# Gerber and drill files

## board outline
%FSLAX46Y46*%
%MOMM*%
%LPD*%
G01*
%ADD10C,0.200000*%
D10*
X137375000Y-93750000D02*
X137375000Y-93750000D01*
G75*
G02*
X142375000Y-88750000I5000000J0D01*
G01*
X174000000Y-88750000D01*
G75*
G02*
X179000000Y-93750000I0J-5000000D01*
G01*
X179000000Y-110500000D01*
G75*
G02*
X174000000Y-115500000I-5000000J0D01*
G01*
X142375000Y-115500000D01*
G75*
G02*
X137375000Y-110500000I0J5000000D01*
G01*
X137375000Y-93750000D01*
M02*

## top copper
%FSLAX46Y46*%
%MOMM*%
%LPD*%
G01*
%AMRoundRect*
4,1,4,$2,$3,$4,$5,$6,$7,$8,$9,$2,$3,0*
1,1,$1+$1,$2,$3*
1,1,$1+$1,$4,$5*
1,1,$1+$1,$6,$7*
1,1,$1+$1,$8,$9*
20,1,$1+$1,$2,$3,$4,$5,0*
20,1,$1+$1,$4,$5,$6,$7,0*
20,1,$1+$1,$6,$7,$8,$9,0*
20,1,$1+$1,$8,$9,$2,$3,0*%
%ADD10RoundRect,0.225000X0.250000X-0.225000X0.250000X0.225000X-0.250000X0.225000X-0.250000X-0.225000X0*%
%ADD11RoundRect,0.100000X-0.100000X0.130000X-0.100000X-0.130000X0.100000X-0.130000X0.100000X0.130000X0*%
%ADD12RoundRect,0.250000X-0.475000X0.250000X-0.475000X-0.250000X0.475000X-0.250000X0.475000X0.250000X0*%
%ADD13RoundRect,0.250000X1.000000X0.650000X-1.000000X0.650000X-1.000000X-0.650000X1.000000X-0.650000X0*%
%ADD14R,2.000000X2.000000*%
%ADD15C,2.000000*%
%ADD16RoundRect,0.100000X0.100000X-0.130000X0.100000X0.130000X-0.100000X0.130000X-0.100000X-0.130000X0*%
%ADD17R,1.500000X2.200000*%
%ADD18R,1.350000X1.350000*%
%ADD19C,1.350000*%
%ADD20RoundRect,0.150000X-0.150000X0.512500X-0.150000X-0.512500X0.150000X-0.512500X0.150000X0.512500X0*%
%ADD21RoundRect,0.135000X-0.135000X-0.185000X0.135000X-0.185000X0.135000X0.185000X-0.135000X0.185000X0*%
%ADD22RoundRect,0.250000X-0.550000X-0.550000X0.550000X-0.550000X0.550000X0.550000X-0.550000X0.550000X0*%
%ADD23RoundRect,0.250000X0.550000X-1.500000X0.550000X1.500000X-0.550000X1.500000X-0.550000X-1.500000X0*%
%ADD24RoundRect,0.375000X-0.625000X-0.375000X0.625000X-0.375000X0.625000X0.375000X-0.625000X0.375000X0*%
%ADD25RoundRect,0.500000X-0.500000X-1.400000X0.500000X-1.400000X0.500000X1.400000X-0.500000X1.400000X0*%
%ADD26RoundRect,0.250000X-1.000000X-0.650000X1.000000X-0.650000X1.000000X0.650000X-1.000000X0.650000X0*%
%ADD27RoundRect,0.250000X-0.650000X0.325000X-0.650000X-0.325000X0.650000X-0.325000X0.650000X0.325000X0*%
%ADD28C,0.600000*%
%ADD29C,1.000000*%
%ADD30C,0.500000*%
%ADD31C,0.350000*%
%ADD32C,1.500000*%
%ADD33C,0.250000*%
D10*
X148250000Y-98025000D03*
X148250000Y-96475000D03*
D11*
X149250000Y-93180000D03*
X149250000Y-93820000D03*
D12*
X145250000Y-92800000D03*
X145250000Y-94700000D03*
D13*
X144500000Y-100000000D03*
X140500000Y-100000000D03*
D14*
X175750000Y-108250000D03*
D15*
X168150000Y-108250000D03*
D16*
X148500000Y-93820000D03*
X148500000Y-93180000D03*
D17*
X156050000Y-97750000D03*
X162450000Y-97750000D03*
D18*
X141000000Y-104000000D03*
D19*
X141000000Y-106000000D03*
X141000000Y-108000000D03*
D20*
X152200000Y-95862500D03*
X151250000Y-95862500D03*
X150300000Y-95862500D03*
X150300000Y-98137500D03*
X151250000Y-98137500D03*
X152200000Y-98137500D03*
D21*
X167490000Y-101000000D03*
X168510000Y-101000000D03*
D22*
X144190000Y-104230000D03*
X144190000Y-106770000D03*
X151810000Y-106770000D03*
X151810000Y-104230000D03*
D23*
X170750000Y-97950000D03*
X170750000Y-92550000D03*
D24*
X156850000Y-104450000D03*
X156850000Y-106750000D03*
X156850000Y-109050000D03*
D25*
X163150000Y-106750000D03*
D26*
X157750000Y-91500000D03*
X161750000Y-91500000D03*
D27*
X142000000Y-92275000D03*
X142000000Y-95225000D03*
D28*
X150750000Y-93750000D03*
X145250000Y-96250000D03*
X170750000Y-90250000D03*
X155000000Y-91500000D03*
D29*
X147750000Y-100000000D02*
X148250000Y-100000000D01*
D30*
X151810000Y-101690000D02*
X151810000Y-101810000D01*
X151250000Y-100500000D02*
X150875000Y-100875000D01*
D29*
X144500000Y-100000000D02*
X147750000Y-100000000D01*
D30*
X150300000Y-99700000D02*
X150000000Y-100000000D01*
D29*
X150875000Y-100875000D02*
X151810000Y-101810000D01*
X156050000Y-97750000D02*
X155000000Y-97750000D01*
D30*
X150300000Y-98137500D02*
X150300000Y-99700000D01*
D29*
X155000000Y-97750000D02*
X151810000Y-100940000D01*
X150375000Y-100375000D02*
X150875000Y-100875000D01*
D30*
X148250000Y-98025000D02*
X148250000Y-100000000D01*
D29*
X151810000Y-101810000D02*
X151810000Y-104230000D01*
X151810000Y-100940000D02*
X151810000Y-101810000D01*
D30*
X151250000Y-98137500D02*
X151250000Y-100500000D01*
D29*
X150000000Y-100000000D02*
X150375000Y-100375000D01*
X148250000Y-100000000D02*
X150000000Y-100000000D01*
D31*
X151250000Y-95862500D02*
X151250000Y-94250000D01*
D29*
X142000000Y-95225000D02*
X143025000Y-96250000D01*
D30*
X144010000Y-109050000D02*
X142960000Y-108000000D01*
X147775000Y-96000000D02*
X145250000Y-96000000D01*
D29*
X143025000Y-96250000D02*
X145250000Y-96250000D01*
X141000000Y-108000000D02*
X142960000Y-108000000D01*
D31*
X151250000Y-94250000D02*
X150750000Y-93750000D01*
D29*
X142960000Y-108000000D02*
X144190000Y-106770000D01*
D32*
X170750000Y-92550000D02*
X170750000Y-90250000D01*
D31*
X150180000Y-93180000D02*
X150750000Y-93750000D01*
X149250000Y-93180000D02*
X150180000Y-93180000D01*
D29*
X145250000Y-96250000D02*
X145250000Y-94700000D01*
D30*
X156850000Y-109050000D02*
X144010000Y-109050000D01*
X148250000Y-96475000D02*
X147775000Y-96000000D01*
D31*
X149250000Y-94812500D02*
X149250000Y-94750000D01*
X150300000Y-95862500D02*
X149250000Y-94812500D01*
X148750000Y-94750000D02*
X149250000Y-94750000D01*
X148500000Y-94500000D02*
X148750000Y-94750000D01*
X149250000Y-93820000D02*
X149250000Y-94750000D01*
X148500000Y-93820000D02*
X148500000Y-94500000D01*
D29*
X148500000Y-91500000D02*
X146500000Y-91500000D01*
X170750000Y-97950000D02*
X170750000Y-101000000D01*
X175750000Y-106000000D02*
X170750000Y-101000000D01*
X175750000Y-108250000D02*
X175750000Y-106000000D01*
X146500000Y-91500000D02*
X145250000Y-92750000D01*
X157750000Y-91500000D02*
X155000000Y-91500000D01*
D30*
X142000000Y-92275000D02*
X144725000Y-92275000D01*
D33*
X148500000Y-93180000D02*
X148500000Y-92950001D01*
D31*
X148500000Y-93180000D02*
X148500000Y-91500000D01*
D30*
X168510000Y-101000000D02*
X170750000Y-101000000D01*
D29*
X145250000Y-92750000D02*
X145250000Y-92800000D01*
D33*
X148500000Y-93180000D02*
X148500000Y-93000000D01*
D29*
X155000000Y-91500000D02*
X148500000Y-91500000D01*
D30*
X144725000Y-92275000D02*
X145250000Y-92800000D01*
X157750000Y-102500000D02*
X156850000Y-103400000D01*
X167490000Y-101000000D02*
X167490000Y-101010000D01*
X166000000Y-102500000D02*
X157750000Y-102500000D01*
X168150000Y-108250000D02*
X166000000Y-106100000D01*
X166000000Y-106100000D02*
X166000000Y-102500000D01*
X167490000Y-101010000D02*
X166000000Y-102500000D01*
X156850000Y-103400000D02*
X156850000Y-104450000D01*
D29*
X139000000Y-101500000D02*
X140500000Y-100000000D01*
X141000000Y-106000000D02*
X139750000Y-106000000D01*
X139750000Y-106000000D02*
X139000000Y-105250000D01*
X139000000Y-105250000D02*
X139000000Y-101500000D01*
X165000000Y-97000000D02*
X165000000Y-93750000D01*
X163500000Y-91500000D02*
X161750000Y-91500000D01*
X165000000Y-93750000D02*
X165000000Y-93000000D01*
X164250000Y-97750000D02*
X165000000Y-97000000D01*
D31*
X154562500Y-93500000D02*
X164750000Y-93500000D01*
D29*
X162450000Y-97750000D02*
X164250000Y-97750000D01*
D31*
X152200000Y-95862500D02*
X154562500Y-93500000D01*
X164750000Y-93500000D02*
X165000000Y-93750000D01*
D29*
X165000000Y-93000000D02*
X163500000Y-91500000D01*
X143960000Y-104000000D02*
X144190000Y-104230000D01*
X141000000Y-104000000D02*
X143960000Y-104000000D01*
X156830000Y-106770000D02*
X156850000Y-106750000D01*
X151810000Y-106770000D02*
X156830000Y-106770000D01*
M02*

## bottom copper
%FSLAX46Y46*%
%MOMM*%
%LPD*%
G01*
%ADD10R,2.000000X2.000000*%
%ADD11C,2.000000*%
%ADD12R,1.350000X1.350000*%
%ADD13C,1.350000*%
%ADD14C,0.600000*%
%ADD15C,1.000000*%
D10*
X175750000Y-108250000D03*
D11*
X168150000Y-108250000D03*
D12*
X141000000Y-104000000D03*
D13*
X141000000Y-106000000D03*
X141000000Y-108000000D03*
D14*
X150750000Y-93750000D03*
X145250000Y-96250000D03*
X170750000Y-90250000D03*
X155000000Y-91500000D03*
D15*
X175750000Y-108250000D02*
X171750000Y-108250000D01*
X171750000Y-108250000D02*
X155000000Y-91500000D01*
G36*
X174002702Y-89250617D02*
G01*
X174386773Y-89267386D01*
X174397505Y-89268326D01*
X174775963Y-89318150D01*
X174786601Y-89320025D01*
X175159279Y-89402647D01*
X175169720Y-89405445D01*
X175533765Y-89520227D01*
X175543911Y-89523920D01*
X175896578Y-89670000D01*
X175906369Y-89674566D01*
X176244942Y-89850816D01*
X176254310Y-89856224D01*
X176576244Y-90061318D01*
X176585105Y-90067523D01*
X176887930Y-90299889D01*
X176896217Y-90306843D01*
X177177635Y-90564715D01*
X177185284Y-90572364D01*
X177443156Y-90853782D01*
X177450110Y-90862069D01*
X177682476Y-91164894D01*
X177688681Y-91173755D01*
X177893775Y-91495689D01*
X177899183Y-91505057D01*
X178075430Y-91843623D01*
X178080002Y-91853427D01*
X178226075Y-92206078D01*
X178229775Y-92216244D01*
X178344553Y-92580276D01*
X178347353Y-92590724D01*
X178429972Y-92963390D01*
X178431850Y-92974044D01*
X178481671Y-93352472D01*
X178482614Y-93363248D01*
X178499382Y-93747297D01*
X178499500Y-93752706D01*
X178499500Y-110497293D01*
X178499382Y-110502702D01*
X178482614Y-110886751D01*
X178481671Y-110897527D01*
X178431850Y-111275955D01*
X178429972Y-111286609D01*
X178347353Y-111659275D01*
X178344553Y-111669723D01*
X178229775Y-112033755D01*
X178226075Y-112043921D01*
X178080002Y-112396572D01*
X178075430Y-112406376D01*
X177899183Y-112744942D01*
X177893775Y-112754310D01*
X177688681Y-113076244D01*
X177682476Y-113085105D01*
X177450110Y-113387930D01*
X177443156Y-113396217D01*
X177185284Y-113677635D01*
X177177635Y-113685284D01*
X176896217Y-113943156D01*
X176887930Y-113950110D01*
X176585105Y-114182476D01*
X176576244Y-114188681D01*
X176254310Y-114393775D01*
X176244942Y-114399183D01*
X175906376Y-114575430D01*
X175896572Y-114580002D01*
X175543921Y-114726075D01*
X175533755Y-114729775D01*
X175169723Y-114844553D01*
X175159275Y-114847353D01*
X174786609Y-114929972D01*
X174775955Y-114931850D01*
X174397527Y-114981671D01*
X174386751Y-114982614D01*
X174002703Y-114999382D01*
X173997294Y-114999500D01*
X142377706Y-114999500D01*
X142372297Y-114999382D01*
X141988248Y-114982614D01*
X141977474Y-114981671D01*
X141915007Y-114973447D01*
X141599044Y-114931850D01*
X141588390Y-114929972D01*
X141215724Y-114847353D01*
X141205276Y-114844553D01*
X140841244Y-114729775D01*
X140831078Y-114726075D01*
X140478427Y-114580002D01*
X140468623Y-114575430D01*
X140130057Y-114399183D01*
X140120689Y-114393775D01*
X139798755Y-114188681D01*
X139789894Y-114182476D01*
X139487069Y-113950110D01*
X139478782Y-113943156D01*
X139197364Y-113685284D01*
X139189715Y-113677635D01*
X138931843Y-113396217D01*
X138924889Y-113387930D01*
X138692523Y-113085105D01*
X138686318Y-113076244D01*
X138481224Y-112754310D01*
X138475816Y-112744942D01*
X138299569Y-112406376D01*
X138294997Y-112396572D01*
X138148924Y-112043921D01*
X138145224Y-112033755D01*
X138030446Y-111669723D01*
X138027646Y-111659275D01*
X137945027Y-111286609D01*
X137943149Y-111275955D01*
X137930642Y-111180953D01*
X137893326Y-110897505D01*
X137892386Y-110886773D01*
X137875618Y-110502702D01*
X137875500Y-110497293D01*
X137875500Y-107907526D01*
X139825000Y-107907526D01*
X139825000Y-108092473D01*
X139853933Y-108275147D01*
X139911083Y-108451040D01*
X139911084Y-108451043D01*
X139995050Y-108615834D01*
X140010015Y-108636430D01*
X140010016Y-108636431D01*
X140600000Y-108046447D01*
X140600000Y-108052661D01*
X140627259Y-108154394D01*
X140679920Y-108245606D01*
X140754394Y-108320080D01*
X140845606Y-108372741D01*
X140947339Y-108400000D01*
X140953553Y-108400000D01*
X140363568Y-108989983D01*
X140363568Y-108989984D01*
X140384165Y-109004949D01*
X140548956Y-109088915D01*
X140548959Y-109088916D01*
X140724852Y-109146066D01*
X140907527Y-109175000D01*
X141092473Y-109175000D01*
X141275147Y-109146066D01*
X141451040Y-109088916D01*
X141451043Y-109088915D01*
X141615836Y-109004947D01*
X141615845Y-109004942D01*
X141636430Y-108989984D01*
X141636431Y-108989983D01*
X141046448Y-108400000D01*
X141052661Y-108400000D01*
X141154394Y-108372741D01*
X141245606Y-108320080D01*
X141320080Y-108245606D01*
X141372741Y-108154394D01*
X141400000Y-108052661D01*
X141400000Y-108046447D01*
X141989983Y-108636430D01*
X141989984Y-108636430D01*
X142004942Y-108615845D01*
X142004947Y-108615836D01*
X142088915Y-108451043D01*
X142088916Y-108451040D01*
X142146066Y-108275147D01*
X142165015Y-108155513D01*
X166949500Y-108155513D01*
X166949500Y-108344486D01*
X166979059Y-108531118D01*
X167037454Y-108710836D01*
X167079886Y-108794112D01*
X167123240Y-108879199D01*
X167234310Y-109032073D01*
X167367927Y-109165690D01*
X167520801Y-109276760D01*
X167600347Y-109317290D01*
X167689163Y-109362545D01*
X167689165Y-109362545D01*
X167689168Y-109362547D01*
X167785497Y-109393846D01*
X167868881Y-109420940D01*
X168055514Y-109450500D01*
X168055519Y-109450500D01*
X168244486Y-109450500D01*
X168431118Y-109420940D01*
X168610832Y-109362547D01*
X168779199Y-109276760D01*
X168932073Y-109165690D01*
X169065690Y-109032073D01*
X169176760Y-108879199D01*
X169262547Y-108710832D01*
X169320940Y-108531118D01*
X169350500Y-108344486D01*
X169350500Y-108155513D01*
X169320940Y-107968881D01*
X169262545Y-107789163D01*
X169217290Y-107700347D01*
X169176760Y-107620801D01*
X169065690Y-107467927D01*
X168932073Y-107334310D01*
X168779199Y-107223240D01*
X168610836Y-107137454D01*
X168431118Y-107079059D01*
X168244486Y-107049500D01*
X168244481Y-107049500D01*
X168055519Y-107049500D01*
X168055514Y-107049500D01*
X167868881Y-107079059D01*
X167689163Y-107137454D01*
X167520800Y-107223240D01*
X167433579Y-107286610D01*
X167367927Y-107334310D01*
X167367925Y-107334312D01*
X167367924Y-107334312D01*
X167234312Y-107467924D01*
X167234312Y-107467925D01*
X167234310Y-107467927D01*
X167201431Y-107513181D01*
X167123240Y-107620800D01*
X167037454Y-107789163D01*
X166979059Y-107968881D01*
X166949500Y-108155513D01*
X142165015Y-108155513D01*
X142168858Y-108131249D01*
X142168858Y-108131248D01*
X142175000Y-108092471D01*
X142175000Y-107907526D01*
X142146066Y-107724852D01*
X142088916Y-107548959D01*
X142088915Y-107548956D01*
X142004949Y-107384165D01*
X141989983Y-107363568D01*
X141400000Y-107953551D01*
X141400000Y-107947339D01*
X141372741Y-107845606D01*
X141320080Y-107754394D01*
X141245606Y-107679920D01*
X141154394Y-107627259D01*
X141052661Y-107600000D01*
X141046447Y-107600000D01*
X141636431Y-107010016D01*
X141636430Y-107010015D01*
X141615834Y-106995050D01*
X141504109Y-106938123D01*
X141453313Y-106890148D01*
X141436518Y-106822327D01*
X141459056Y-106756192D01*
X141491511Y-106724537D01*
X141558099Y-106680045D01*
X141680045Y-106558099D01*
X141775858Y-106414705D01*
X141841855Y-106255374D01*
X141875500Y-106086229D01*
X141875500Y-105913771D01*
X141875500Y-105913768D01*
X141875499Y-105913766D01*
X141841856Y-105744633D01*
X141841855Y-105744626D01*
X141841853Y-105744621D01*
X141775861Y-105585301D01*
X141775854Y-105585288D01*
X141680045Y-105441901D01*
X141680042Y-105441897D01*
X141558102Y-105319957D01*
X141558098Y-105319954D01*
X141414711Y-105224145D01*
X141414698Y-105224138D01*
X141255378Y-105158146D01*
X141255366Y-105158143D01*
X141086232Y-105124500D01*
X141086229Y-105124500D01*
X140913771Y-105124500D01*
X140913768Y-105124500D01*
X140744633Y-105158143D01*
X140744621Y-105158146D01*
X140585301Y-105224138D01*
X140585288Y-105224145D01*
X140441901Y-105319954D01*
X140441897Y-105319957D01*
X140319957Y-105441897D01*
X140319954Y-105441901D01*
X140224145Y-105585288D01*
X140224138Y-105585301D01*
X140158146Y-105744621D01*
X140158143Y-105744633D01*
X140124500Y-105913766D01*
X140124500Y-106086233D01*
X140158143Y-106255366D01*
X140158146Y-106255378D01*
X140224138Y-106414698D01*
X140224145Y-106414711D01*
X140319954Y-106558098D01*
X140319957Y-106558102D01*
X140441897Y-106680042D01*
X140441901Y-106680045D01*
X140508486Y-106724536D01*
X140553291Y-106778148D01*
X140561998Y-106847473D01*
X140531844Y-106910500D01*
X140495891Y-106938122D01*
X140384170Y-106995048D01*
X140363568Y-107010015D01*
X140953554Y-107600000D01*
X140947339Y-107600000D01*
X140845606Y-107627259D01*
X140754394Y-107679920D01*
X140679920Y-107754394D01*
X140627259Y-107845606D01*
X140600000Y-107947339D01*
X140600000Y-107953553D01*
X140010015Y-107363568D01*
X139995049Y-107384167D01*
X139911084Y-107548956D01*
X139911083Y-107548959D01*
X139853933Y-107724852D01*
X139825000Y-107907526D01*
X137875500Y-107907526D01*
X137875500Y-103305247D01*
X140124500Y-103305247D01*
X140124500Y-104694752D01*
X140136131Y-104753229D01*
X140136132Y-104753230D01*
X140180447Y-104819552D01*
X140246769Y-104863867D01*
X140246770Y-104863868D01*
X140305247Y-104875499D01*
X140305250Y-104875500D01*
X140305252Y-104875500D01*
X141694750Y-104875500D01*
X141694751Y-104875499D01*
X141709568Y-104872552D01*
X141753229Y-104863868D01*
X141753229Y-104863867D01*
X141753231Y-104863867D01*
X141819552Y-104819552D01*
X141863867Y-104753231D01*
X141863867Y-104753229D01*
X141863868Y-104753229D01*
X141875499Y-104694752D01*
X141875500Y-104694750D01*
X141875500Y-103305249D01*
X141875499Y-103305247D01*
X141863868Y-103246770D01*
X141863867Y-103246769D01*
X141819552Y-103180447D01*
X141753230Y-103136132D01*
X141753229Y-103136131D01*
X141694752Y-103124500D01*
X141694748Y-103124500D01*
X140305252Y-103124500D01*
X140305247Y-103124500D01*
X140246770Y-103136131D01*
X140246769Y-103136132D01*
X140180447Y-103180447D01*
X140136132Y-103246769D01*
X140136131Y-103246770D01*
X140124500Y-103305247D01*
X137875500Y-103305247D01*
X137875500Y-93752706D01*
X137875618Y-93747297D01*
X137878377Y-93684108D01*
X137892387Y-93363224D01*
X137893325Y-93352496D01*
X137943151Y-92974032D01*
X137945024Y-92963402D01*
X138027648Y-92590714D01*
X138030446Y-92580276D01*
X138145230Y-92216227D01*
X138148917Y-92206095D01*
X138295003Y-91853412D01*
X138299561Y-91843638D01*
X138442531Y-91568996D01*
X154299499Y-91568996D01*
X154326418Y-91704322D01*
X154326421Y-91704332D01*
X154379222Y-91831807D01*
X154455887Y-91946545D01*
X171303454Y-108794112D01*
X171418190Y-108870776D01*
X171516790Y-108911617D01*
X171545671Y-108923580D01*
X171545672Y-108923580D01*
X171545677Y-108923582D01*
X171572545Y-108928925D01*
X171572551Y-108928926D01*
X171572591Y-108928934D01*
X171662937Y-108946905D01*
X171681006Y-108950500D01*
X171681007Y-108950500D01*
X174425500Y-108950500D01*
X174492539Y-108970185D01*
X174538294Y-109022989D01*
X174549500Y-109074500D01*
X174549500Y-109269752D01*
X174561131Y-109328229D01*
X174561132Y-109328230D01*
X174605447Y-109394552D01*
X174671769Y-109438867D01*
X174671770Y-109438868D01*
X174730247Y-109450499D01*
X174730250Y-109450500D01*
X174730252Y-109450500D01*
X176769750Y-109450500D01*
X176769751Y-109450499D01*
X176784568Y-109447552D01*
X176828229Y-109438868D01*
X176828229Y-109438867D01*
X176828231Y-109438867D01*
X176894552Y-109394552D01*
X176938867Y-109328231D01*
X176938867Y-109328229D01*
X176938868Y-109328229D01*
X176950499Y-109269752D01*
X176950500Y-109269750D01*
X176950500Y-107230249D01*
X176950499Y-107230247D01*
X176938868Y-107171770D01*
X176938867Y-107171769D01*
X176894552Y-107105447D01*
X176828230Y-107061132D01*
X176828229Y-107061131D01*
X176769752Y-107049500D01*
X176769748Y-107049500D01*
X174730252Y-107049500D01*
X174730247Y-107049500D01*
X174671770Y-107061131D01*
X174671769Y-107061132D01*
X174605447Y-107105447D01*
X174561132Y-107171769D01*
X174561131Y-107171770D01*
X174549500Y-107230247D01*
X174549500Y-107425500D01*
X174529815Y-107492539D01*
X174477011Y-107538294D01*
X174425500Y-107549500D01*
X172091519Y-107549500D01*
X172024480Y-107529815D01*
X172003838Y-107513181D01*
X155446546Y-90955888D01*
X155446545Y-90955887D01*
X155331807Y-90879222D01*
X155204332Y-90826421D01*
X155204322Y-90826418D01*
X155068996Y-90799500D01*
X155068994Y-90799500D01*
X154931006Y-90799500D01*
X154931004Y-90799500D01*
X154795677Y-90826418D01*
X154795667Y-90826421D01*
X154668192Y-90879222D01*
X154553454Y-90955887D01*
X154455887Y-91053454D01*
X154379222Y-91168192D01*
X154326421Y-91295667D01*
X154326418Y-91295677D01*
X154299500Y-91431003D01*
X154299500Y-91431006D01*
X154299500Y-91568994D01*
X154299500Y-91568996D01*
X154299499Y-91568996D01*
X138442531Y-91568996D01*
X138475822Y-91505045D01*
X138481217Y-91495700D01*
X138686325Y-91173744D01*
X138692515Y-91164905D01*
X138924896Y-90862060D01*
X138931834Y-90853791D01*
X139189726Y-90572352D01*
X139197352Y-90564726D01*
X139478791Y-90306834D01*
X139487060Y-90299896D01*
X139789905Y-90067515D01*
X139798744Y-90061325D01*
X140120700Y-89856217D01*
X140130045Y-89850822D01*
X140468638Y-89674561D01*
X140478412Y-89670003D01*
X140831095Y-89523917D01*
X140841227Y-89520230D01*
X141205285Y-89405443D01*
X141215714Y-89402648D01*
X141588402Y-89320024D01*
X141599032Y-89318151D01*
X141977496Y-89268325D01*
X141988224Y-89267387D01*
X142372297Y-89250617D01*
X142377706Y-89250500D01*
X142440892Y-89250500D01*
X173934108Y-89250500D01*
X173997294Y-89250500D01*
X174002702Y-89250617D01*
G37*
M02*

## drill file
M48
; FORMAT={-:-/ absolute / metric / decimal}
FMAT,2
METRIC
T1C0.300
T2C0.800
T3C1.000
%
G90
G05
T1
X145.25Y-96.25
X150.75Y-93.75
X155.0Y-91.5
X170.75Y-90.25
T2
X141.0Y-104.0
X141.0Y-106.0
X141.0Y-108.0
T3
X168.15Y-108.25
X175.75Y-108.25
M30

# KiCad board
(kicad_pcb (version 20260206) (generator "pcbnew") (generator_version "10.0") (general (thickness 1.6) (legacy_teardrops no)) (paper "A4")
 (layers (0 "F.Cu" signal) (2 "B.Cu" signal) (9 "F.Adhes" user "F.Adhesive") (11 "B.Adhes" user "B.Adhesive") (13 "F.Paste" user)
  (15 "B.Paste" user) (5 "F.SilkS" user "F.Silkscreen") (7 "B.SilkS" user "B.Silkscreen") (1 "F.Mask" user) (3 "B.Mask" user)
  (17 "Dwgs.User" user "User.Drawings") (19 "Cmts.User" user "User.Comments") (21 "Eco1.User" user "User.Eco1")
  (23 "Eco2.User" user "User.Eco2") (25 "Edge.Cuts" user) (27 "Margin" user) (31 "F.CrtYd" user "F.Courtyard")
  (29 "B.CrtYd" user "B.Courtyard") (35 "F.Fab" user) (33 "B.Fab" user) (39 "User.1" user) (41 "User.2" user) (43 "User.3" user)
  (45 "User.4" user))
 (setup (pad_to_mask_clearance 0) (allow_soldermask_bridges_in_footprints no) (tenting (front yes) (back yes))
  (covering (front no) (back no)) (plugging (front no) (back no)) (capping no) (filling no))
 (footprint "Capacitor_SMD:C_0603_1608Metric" (layer "F.Cu") (at 148.25 97.25 90)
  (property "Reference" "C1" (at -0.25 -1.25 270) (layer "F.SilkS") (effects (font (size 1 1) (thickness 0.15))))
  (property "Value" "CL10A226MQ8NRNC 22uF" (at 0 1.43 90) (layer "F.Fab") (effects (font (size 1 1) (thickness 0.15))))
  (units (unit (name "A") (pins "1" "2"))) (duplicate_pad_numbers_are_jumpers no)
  (pad "1" smd roundrect (at -0.775 0 90) (size 0.9 0.95) (layers "F.Cu" "F.Mask" "F.Paste") (roundrect_rratio 0.25) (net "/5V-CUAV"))
  (pad "2" smd roundrect (at 0.775 0 90) (size 0.9 0.95) (layers "F.Cu" "F.Mask" "F.Paste") (roundrect_rratio 0.25) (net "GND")))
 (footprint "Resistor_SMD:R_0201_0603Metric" (layer "F.Cu") (at 149.25 93.5 -90)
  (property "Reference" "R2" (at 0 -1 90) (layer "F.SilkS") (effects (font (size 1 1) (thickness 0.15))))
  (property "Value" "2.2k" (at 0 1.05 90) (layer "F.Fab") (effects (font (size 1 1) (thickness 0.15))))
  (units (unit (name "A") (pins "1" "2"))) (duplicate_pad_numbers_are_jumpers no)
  (pad "" smd roundrect (at -0.345 0 270) (size 0.318 0.36) (layers "F.Paste") (roundrect_rratio 0.25))
  (pad "" smd roundrect (at 0.345 0 270) (size 0.318 0.36) (layers "F.Paste") (roundrect_rratio 0.25))
  (pad "1" smd roundrect (at -0.32 0 270) (size 0.46 0.4) (layers "F.Cu" "F.Mask") (roundrect_rratio 0.25) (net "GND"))
  (pad "2" smd roundrect (at 0.32 0 270) (size 0.46 0.4) (layers "F.Cu" "F.Mask") (roundrect_rratio 0.25) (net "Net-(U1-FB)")))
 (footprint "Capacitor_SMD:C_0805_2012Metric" (layer "F.Cu") (at 145.25 93.75 -90)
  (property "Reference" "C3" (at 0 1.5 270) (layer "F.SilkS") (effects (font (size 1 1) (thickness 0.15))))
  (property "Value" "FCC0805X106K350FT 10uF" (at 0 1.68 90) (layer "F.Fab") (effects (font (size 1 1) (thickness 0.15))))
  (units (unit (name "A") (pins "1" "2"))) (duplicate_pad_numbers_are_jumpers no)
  (pad "1" smd roundrect (at -0.95 0 270) (size 1 1.45) (layers "F.Cu" "F.Mask" "F.Paste") (roundrect_rratio 0.25) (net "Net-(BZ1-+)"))
  (pad "2" smd roundrect (at 0.95 0 270) (size 1 1.45) (layers "F.Cu" "F.Mask" "F.Paste") (roundrect_rratio 0.25) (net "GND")))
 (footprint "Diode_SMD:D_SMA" (layer "F.Cu") (at 142.5 100 180)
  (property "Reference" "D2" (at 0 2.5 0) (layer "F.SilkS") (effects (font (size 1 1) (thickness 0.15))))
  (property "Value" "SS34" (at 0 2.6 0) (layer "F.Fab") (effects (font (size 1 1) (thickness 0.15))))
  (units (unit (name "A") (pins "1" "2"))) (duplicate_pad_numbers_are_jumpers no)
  (pad "1" smd roundrect (at -2 0 180) (size 2.5 1.8) (layers "F.Cu" "F.Mask" "F.Paste") (roundrect_rratio 0.1388888889) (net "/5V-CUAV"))
  (pad "2" smd roundrect (at 2 0 180) (size 2.5 1.8) (layers "F.Cu" "F.Mask" "F.Paste") (roundrect_rratio 0.1388888889) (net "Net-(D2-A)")))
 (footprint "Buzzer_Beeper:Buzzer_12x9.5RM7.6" (layer "F.Cu") (at 175.75 108.25 180)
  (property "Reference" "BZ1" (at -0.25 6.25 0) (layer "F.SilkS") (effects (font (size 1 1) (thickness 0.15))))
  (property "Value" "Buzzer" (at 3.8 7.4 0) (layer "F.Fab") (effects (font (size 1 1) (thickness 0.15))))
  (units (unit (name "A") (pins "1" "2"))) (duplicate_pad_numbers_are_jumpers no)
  (pad "1" thru_hole rect (at 0 0 180) (size 2 2) (drill 1) (layers "*.Cu" "*.Mask") (remove_unused_layers no) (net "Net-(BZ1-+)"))
  (pad "2" thru_hole circle (at 7.6 0 180) (size 2 2) (drill 1) (layers "*.Cu" "*.Mask") (remove_unused_layers no) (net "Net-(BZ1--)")))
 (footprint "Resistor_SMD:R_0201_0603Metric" (layer "F.Cu") (at 148.5 93.5 90)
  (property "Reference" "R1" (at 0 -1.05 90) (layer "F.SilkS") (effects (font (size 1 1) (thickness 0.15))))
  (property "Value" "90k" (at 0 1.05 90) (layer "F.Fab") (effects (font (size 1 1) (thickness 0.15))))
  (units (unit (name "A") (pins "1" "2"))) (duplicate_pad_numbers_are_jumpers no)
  (pad "" smd roundrect (at -0.345 0 90) (size 0.318 0.36) (layers "F.Paste") (roundrect_rratio 0.25))
  (pad "" smd roundrect (at 0.345 0 90) (size 0.318 0.36) (layers "F.Paste") (roundrect_rratio 0.25))
  (pad "1" smd roundrect (at -0.32 0 90) (size 0.46 0.4) (layers "F.Cu" "F.Mask") (roundrect_rratio 0.25) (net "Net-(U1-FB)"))
  (pad "2" smd roundrect (at 0.32 0 90) (size 0.46 0.4) (layers "F.Cu" "F.Mask") (roundrect_rratio 0.25) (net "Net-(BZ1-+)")))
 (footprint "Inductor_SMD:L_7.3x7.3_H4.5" (layer "F.Cu") (at 159.25 97.75)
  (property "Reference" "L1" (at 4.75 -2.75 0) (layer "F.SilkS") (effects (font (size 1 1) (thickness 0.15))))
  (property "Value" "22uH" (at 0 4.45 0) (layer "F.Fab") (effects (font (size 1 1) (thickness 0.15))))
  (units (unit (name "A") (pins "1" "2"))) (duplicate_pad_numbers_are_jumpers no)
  (pad "1" smd rect (at -3.2 0) (size 1.5 2.2) (layers "F.Cu" "F.Mask" "F.Paste") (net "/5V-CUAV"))
  (pad "2" smd rect (at 3.2 0) (size 1.5 2.2) (layers "F.Cu" "F.Mask" "F.Paste") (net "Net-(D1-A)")))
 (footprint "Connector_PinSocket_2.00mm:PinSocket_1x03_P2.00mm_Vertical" (layer "F.Cu") (at 141 104)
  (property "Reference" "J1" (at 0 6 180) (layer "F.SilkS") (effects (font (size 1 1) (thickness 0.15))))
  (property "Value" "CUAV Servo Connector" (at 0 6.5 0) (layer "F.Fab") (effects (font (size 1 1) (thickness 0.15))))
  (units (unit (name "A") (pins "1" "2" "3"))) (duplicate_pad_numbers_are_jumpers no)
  (pad "1" thru_hole rect (at 0 0) (size 1.35 1.35) (drill 0.8) (layers "*.Cu" "*.Mask") (remove_unused_layers no) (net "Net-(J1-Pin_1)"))
  (pad "2" thru_hole circle (at 0 2) (size 1.35 1.35) (drill 0.8) (layers "*.Cu" "*.Mask") (remove_unused_layers no) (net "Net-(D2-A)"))
  (pad "3" thru_hole circle (at 0 4) (size 1.35 1.35) (drill 0.8) (layers "*.Cu" "*.Mask") (remove_unused_layers no) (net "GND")))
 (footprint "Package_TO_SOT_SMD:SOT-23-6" (layer "F.Cu") (at 151.25 97 -90)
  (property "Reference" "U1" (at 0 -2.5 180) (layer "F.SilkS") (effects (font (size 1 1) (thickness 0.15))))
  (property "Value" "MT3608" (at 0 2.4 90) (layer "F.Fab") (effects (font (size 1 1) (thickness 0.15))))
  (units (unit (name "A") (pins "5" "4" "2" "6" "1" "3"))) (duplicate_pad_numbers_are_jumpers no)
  (pad "1" smd roundrect (at -1.1375 -0.95 270) (size 1.325 0.6) (layers "F.Cu" "F.Mask" "F.Paste") (roundrect_rratio 0.25)
   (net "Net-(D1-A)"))
  (pad "2" smd roundrect (at -1.1375 0 270) (size 1.325 0.6) (layers "F.Cu" "F.Mask" "F.Paste") (roundrect_rratio 0.25) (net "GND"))
  (pad "3" smd roundrect (at -1.1375 0.95 270) (size 1.325 0.6) (layers "F.Cu" "F.Mask" "F.Paste") (roundrect_rratio 0.25)
   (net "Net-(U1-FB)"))
  (pad "4" smd roundrect (at 1.1375 0.95 270) (size 1.325 0.6) (layers "F.Cu" "F.Mask" "F.Paste") (roundrect_rratio 0.25) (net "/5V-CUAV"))
  (pad "5" smd roundrect (at 1.1375 0 270) (size 1.325 0.6) (layers "F.Cu" "F.Mask" "F.Paste") (roundrect_rratio 0.25) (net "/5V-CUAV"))
  (pad "6" smd roundrect (at 1.1375 -0.95 270) (size 1.325 0.6) (layers "F.Cu" "F.Mask" "F.Paste") (roundrect_rratio 0.25)
   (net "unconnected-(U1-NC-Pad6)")))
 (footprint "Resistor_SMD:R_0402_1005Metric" (layer "F.Cu") (at 168 101)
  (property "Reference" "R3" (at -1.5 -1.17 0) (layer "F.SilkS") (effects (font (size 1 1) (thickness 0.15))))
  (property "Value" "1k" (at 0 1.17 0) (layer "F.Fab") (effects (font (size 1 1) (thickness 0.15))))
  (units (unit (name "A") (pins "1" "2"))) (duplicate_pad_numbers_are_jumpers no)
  (pad "1" smd roundrect (at -0.51 0) (size 0.54 0.64) (layers "F.Cu" "F.Mask" "F.Paste") (roundrect_rratio 0.25) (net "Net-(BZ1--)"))
  (pad "2" smd roundrect (at 0.51 0) (size 0.54 0.64) (layers "F.Cu" "F.Mask" "F.Paste") (roundrect_rratio 0.25) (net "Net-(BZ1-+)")))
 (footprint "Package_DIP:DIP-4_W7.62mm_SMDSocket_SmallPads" (layer "F.Cu") (at 148 105.5)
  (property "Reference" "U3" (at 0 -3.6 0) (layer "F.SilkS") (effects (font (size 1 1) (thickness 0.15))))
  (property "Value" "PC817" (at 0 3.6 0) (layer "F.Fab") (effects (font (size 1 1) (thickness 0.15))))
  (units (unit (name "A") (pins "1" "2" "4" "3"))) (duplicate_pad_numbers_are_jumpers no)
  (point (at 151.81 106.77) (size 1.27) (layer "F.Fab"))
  (pad "1" smd roundrect (at -3.81 -1.27) (size 1.6 1.6) (layers "F.Cu" "F.Mask" "F.Paste") (roundrect_rratio 0.15625)
   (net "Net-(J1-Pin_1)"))
  (pad "2" smd roundrect (at -3.81 1.27) (size 1.6 1.6) (layers "F.Cu" "F.Mask" "F.Paste") (roundrect_rratio 0.15625) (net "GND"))
  (pad "3" smd roundrect (at 3.81 1.27) (size 1.6 1.6) (layers "F.Cu" "F.Mask" "F.Paste") (roundrect_rratio 0.15625) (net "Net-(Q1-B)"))
  (pad "4" smd roundrect (at 3.81 -1.27) (size 1.6 1.6) (layers "F.Cu" "F.Mask" "F.Paste") (roundrect_rratio 0.15625) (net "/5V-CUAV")))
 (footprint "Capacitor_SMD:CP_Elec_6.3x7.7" (layer "F.Cu") (at 170.75 95.25 90)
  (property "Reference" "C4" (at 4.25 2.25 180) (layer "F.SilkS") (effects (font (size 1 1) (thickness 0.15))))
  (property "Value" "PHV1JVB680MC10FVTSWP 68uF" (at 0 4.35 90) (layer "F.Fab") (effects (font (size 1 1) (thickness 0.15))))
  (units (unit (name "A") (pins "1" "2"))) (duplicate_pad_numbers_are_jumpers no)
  (pad "1" smd roundrect (at -2.7 0 90) (size 3.5 1.6) (layers "F.Cu" "F.Mask" "F.Paste") (roundrect_rratio 0.15625) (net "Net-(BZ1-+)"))
  (pad "2" smd roundrect (at 2.7 0 90) (size 3.5 1.6) (layers "F.Cu" "F.Mask" "F.Paste") (roundrect_rratio 0.15625) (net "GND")))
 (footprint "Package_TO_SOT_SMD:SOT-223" (layer "F.Cu") (at 160 106.75)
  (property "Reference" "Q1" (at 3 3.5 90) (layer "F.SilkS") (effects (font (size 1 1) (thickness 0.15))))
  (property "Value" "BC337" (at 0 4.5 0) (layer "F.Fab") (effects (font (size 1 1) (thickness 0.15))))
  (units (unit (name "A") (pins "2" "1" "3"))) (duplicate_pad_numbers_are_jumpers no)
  (pad "1" smd roundrect (at -3.15 -2.3) (size 2 1.5) (layers "F.Cu" "F.Mask" "F.Paste") (roundrect_rratio 0.25) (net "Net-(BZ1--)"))
  (pad "2" smd roundrect (at -3.15 0) (size 2 1.5) (layers "F.Cu" "F.Mask" "F.Paste") (roundrect_rratio 0.25) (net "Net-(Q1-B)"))
  (pad "3" smd roundrect (at -3.15 2.3) (size 2 1.5) (layers "F.Cu" "F.Mask" "F.Paste") (roundrect_rratio 0.25) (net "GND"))
  (pad "4" smd roundrect (at 3.15 0) (size 2 3.8) (layers "F.Cu" "F.Mask" "F.Paste") (roundrect_rratio 0.25)))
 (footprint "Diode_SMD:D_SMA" (layer "F.Cu") (at 159.75 91.5)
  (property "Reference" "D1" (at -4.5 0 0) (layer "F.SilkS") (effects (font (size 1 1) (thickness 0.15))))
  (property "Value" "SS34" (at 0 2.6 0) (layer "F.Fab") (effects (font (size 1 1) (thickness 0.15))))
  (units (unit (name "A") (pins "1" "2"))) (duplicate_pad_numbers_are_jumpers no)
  (pad "1" smd roundrect (at -2 0) (size 2.5 1.8) (layers "F.Cu" "F.Mask" "F.Paste") (roundrect_rratio 0.1388888889) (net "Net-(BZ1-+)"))
  (pad "2" smd roundrect (at 2 0) (size 2.5 1.8) (layers "F.Cu" "F.Mask" "F.Paste") (roundrect_rratio 0.1388888889) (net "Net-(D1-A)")))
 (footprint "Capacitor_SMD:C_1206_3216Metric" (layer "F.Cu") (at 142 93.75 -90)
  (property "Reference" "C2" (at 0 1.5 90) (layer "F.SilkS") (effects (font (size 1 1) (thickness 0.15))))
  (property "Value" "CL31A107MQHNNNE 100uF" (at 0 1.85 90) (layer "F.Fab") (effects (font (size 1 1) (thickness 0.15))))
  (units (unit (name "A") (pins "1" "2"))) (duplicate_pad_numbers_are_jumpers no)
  (pad "1" smd roundrect (at -1.475 0 270) (size 1.15 1.8) (layers "F.Cu" "F.Mask" "F.Paste") (roundrect_rratio 0.217391)
   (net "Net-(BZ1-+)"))
  (pad "2" smd roundrect (at 1.475 0 270) (size 1.15 1.8) (layers "F.Cu" "F.Mask" "F.Paste") (roundrect_rratio 0.217391) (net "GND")))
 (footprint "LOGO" (layer "B.Cu") (at 159.192343 103.04079 180)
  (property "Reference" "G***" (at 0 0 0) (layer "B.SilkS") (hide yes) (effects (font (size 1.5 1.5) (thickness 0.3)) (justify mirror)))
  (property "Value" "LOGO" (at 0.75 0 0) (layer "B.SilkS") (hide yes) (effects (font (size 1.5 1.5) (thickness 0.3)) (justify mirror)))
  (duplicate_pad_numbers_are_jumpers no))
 (gr_rect (start 137.375 88.75) (end 179 115.5) (radius 5) (stroke (width 0.2) (type solid)) (fill no) (layer "Edge.Cuts"))
 (segment (start 147.75 100) (end 148.25 100) (width 1) (layer "F.Cu") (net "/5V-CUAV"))
 (segment (start 151.81 101.69) (end 151.81 101.81) (width 0.5) (layer "F.Cu") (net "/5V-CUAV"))
 (segment (start 151.25 100.5) (end 150.875 100.875) (width 0.5) (layer "F.Cu") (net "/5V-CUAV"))
 (segment (start 144.5 100) (end 147.75 100) (width 1) (layer "F.Cu") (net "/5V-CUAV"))
 (segment (start 150.3 99.7) (end 150 100) (width 0.5) (layer "F.Cu") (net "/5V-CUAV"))
 (segment (start 150.875 100.875) (end 151.81 101.81) (width 1) (layer "F.Cu") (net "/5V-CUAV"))
 (segment (start 156.05 97.75) (end 155 97.75) (width 1) (layer "F.Cu") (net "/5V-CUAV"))
 (segment (start 150.3 98.1375) (end 150.3 99.7) (width 0.5) (layer "F.Cu") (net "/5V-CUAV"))
 (segment (start 155 97.75) (end 151.81 100.94) (width 1) (layer "F.Cu") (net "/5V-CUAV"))
 (segment (start 150.375 100.375) (end 150.875 100.875) (width 1) (layer "F.Cu") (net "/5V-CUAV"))
 (segment (start 148.25 98.025) (end 148.25 100) (width 0.5) (layer "F.Cu") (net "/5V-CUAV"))
 (segment (start 151.81 101.81) (end 151.81 104.23) (width 1) (layer "F.Cu") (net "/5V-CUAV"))
 (segment (start 151.81 100.94) (end 151.81 101.81) (width 1) (layer "F.Cu") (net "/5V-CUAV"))
 (segment (start 151.25 98.1375) (end 151.25 100.5) (width 0.5) (layer "F.Cu") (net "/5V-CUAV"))
 (segment (start 150 100) (end 150.375 100.375) (width 1) (layer "F.Cu") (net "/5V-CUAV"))
 (segment (start 148.25 100) (end 150 100) (width 1) (layer "F.Cu") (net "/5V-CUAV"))
 (segment (start 151.25 95.8625) (end 151.25 94.25) (width 0.35) (layer "F.Cu") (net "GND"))
 (segment (start 142 95.225) (end 143.025 96.25) (width 1) (layer "F.Cu") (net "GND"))
 (segment (start 144.01 109.05) (end 142.96 108) (width 0.5) (layer "F.Cu") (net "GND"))
 (segment (start 147.775 96) (end 145.25 96) (width 0.5) (layer "F.Cu") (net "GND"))
 (segment (start 143.025 96.25) (end 145.25 96.25) (width 1) (layer "F.Cu") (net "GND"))
 (segment (start 141 108) (end 142.96 108) (width 1) (layer "F.Cu") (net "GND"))
 (segment (start 151.25 94.25) (end 150.75 93.75) (width 0.35) (layer "F.Cu") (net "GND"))
 (segment (start 142.96 108) (end 144.19 106.77) (width 1) (layer "F.Cu") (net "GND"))
 (segment (start 170.75 92.55) (end 170.75 90.25) (width 1.5) (layer "F.Cu") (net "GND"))
 (segment (start 150.18 93.18) (end 150.75 93.75) (width 0.35) (layer "F.Cu") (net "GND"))
 (segment (start 149.25 93.18) (end 150.18 93.18) (width 0.35) (layer "F.Cu") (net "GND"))
 (segment (start 145.25 96.25) (end 145.25 94.7) (width 1) (layer "F.Cu") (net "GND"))
 (segment (start 156.85 109.05) (end 144.01 109.05) (width 0.5) (layer "F.Cu") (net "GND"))
 (segment (start 148.25 96.475) (end 147.775 96) (width 0.5) (layer "F.Cu") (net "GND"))
 (via (at 150.75 93.75) (size 0.6) (drill 0.3) (layers "F.Cu" "B.Cu") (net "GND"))
 (via (at 145.25 96.25) (size 0.6) (drill 0.3) (layers "F.Cu" "B.Cu") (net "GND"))
 (via (at 170.75 90.25) (size 0.6) (drill 0.3) (layers "F.Cu" "B.Cu") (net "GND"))
 (segment (start 149.25 94.8125) (end 149.25 94.75) (width 0.35) (layer "F.Cu") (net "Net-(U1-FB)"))
 (segment (start 150.3 95.8625) (end 149.25 94.8125) (width 0.35) (layer "F.Cu") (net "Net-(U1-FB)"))
 (segment (start 148.75 94.75) (end 149.25 94.75) (width 0.35) (layer "F.Cu") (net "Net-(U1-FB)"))
 (segment (start 148.5 94.5) (end 148.75 94.75) (width 0.35) (layer "F.Cu") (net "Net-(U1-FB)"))
 (segment (start 149.25 93.82) (end 149.25 94.75) (width 0.35) (layer "F.Cu") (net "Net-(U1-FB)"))
 (segment (start 148.5 93.82) (end 148.5 94.5) (width 0.35) (layer "F.Cu") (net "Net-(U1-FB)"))
 (segment (start 148.5 91.5) (end 146.5 91.5) (width 1) (layer "F.Cu") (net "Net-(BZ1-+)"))
 (segment (start 170.75 97.95) (end 170.75 101) (width 1) (layer "F.Cu") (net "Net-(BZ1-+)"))
 (segment (start 175.75 106) (end 170.75 101) (width 1) (layer "F.Cu") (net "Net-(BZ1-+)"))
 (segment (start 175.75 108.25) (end 175.75 106) (width 1) (layer "F.Cu") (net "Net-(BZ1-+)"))
 (segment (start 146.5 91.5) (end 145.25 92.75) (width 1) (layer "F.Cu") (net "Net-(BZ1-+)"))
 (segment (start 157.75 91.5) (end 155 91.5) (width 1) (layer "F.Cu") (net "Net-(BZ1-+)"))
 (segment (start 142 92.275) (end 144.725 92.275) (width 0.5) (layer "F.Cu") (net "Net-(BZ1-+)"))
 (segment (start 148.5 93.18) (end 148.5 92.950001) (width 0.25) (layer "F.Cu") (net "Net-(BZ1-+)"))
 (segment (start 148.5 93.18) (end 148.5 91.5) (width 0.35) (layer "F.Cu") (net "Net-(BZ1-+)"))
 (segment (start 168.51 101) (end 170.75 101) (width 0.5) (layer "F.Cu") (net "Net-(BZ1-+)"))
 (segment (start 145.25 92.75) (end 145.25 92.8) (width 1) (layer "F.Cu") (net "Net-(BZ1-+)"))
 (segment (start 148.5 93.18) (end 148.5 93) (width 0.25) (layer "F.Cu") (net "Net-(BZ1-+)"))
 (segment (start 155 91.5) (end 148.5 91.5) (width 1) (layer "F.Cu") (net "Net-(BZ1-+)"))
 (segment (start 144.725 92.275) (end 145.25 92.8) (width 0.5) (layer "F.Cu") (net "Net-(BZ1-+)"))
 (via (at 155 91.5) (size 0.6) (drill 0.3) (layers "F.Cu" "B.Cu") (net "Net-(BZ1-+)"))
 (segment (start 175.75 108.25) (end 171.75 108.25) (width 1) (layer "B.Cu") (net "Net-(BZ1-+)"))
 (segment (start 171.75 108.25) (end 155 91.5) (width 1) (layer "B.Cu") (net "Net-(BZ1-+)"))
 (segment (start 157.75 102.5) (end 156.85 103.4) (width 0.5) (layer "F.Cu") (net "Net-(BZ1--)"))
 (segment (start 167.49 101) (end 167.49 101.01) (width 0.5) (layer "F.Cu") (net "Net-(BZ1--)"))
 (segment (start 166 102.5) (end 157.75 102.5) (width 0.5) (layer "F.Cu") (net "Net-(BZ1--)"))
 (segment (start 168.15 108.25) (end 166 106.1) (width 0.5) (layer "F.Cu") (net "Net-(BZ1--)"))
 (segment (start 166 106.1) (end 166 102.5) (width 0.5) (layer "F.Cu") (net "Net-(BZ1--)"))
 (segment (start 167.49 101.01) (end 166 102.5) (width 0.5) (layer "F.Cu") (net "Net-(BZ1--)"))
 (segment (start 156.85 103.4) (end 156.85 104.45) (width 0.5) (layer "F.Cu") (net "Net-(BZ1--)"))
 (segment (start 139 101.5) (end 140.5 100) (width 1) (layer "F.Cu") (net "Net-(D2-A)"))
 (segment (start 141 106) (end 139.75 106) (width 1) (layer "F.Cu") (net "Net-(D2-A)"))
 (segment (start 139.75 106) (end 139 105.25) (width 1) (layer "F.Cu") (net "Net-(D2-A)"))
 (segment (start 139 105.25) (end 139 101.5) (width 1) (layer "F.Cu") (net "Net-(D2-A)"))
 (segment (start 165 97) (end 165 93.75) (width 1) (layer "F.Cu") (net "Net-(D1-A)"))
 (segment (start 163.5 91.5) (end 161.75 91.5) (width 1) (layer "F.Cu") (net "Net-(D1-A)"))
 (segment (start 165 93.75) (end 165 93) (width 1) (layer "F.Cu") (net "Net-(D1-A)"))
 (segment (start 164.25 97.75) (end 165 97) (width 1) (layer "F.Cu") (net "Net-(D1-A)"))
 (segment (start 154.5625 93.5) (end 164.75 93.5) (width 0.35) (layer "F.Cu") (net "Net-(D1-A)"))
 (segment (start 162.45 97.75) (end 164.25 97.75) (width 1) (layer "F.Cu") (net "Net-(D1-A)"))
 (segment (start 152.2 95.8625) (end 154.5625 93.5) (width 0.35) (layer "F.Cu") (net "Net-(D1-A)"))
 (segment (start 164.75 93.5) (end 165 93.75) (width 0.35) (layer "F.Cu") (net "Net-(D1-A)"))
 (segment (start 165 93) (end 163.5 91.5) (width 1) (layer "F.Cu") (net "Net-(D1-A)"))
 (segment (start 143.96 104) (end 144.19 104.23) (width 1) (layer "F.Cu") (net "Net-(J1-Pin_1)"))
 (segment (start 141 104) (end 143.96 104) (width 1) (layer "F.Cu") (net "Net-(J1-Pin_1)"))
 (segment (start 156.83 106.77) (end 156.85 106.75) (width 1) (layer "F.Cu") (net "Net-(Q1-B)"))
 (segment (start 151.81 106.77) (end 156.83 106.77) (width 1) (layer "F.Cu") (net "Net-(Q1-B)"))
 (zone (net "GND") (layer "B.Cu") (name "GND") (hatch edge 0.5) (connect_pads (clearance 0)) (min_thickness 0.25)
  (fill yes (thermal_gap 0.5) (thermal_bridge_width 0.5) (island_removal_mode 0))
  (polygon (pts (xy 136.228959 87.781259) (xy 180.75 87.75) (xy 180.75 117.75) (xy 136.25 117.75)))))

